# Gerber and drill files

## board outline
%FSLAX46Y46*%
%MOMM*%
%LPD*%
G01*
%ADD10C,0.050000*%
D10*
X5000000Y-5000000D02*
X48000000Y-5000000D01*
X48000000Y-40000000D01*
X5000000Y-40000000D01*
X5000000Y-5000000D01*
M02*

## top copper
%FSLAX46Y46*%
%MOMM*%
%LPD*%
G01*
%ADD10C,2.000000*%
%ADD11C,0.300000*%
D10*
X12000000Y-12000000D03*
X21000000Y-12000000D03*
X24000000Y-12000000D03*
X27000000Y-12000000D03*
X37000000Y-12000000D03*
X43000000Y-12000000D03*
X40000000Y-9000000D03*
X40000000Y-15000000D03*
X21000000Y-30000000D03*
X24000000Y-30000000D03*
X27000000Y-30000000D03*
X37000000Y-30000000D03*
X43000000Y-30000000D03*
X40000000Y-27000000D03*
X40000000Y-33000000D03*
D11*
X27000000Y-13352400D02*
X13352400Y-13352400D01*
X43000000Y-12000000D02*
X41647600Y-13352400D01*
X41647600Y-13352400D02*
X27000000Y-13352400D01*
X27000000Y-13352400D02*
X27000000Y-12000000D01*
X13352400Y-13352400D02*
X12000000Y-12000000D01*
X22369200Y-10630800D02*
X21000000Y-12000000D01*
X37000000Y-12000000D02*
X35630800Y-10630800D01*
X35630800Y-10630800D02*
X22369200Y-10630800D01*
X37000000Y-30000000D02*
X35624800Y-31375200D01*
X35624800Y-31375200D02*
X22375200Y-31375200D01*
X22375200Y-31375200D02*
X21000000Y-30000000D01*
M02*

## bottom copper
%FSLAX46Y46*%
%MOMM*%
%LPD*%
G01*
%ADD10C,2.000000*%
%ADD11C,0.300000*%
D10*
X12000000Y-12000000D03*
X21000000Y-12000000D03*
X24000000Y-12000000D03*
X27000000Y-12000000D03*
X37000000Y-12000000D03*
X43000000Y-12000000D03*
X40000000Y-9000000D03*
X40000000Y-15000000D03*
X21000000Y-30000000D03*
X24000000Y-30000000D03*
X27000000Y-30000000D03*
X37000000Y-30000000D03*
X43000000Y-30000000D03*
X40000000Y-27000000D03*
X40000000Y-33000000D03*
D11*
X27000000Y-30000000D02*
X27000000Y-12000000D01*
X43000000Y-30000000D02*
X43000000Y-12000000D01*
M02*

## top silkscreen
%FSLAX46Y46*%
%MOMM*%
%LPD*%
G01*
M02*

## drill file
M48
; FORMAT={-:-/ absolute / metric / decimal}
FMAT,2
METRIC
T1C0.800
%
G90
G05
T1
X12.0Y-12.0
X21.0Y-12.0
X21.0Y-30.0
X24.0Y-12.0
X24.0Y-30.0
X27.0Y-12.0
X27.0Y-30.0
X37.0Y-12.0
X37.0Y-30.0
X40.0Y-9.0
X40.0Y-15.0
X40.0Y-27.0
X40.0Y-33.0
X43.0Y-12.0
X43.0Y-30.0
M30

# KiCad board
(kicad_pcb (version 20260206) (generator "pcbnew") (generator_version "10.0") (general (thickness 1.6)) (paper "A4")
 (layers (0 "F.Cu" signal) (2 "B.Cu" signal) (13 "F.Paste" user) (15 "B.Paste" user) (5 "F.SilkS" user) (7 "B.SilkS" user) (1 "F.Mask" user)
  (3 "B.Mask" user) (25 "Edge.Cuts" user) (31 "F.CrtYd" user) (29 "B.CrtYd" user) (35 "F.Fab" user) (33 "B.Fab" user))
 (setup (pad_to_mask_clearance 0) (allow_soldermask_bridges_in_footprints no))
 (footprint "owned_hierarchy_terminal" (layer "F.Cu") (at 12 12)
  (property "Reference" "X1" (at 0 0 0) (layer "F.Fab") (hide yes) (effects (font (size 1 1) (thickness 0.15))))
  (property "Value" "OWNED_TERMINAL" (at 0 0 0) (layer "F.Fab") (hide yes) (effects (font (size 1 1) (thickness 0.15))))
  (pad "1" thru_hole circle (at 0 0) (size 2 2) (drill 0.8) (layers "*.Cu" "*.Mask") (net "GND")))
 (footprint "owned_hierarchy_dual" (layer "F.Cu") (at 24 12)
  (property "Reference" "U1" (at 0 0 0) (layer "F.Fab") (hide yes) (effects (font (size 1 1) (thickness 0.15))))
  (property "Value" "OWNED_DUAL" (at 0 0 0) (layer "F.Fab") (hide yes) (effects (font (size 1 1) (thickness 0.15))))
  (pad "1" thru_hole circle (at -3 0) (size 2 2) (drill 0.8) (layers "*.Cu" "*.Mask") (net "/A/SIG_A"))
  (pad "2" thru_hole circle (at 0 0) (size 2 2) (drill 0.8) (layers "*.Cu" "*.Mask") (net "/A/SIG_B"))
  (pad "3" thru_hole circle (at 3 0) (size 2 2) (drill 0.8) (layers "*.Cu" "*.Mask") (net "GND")))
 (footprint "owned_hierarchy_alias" (layer "F.Cu") (at 40 12)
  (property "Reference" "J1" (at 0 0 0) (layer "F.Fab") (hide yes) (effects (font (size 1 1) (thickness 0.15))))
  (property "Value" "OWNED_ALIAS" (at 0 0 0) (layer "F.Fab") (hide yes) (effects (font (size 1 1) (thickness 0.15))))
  (pad "R" thru_hole circle (at -3 0) (size 2 2) (drill 0.8) (layers "*.Cu" "*.Mask") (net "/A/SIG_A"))
  (pad "T" thru_hole circle (at 3 0) (size 2 2) (drill 0.8) (layers "*.Cu" "*.Mask") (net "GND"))
  (pad "MP" thru_hole circle (at 0 -3) (size 2 2) (drill 0.8) (layers "*.Cu" "*.Mask"))
  (pad "MP" thru_hole circle (at 0 3) (size 2 2) (drill 0.8) (layers "*.Cu" "*.Mask")))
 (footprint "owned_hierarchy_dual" (layer "F.Cu") (at 24 30)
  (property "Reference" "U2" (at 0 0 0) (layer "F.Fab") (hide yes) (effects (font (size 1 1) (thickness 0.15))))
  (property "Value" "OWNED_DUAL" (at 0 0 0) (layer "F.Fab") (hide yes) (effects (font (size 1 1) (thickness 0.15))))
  (pad "1" thru_hole circle (at -3 0) (size 2 2) (drill 0.8) (layers "*.Cu" "*.Mask") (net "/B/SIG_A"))
  (pad "2" thru_hole circle (at 0 0) (size 2 2) (drill 0.8) (layers "*.Cu" "*.Mask") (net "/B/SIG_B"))
  (pad "3" thru_hole circle (at 3 0) (size 2 2) (drill 0.8) (layers "*.Cu" "*.Mask") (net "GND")))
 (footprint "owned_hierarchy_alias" (layer "F.Cu") (at 40 30)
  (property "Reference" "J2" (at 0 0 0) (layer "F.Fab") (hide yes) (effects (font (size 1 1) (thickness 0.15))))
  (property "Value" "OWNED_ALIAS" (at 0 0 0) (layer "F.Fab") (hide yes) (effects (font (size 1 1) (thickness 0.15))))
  (pad "R" thru_hole circle (at -3 0) (size 2 2) (drill 0.8) (layers "*.Cu" "*.Mask") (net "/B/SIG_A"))
  (pad "T" thru_hole circle (at 3 0) (size 2 2) (drill 0.8) (layers "*.Cu" "*.Mask") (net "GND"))
  (pad "MP" thru_hole circle (at 0 -3) (size 2 2) (drill 0.8) (layers "*.Cu" "*.Mask"))
  (pad "MP" thru_hole circle (at 0 3) (size 2 2) (drill 0.8) (layers "*.Cu" "*.Mask")))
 (gr_rect (start 5 5) (end 48 40) (stroke (width 0.05) (type default)) (fill none) (layer "Edge.Cuts"))
 (segment (start 27 13.3524) (end 13.3524 13.3524) (width 0.3) (layer "F.Cu") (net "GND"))
 (segment (start 43 12) (end 41.6476 13.3524) (width 0.3) (layer "F.Cu") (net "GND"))
 (segment (start 41.6476 13.3524) (end 27 13.3524) (width 0.3) (layer "F.Cu") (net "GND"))
 (segment (start 27 13.3524) (end 27 12) (width 0.3) (layer "F.Cu") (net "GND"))
 (segment (start 13.3524 13.3524) (end 12 12) (width 0.3) (layer "F.Cu") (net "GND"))
 (segment (start 27 30) (end 27 12) (width 0.3) (layer "B.Cu") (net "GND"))
 (segment (start 43 30) (end 43 12) (width 0.3) (layer "B.Cu") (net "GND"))
 (segment (start 22.3692 10.6308) (end 21 12) (width 0.3) (layer "F.Cu") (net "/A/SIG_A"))
 (segment (start 37 12) (end 35.6308 10.6308) (width 0.3) (layer "F.Cu") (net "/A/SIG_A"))
 (segment (start 35.6308 10.6308) (end 22.3692 10.6308) (width 0.3) (layer "F.Cu") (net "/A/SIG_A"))
 (segment (start 37 30) (end 35.6248 31.3752) (width 0.3) (layer "F.Cu") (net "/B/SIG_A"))
 (segment (start 35.6248 31.3752) (end 22.3752 31.3752) (width 0.3) (layer "F.Cu") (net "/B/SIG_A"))
 (segment (start 22.3752 31.3752) (end 21 30) (width 0.3) (layer "F.Cu") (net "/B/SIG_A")))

